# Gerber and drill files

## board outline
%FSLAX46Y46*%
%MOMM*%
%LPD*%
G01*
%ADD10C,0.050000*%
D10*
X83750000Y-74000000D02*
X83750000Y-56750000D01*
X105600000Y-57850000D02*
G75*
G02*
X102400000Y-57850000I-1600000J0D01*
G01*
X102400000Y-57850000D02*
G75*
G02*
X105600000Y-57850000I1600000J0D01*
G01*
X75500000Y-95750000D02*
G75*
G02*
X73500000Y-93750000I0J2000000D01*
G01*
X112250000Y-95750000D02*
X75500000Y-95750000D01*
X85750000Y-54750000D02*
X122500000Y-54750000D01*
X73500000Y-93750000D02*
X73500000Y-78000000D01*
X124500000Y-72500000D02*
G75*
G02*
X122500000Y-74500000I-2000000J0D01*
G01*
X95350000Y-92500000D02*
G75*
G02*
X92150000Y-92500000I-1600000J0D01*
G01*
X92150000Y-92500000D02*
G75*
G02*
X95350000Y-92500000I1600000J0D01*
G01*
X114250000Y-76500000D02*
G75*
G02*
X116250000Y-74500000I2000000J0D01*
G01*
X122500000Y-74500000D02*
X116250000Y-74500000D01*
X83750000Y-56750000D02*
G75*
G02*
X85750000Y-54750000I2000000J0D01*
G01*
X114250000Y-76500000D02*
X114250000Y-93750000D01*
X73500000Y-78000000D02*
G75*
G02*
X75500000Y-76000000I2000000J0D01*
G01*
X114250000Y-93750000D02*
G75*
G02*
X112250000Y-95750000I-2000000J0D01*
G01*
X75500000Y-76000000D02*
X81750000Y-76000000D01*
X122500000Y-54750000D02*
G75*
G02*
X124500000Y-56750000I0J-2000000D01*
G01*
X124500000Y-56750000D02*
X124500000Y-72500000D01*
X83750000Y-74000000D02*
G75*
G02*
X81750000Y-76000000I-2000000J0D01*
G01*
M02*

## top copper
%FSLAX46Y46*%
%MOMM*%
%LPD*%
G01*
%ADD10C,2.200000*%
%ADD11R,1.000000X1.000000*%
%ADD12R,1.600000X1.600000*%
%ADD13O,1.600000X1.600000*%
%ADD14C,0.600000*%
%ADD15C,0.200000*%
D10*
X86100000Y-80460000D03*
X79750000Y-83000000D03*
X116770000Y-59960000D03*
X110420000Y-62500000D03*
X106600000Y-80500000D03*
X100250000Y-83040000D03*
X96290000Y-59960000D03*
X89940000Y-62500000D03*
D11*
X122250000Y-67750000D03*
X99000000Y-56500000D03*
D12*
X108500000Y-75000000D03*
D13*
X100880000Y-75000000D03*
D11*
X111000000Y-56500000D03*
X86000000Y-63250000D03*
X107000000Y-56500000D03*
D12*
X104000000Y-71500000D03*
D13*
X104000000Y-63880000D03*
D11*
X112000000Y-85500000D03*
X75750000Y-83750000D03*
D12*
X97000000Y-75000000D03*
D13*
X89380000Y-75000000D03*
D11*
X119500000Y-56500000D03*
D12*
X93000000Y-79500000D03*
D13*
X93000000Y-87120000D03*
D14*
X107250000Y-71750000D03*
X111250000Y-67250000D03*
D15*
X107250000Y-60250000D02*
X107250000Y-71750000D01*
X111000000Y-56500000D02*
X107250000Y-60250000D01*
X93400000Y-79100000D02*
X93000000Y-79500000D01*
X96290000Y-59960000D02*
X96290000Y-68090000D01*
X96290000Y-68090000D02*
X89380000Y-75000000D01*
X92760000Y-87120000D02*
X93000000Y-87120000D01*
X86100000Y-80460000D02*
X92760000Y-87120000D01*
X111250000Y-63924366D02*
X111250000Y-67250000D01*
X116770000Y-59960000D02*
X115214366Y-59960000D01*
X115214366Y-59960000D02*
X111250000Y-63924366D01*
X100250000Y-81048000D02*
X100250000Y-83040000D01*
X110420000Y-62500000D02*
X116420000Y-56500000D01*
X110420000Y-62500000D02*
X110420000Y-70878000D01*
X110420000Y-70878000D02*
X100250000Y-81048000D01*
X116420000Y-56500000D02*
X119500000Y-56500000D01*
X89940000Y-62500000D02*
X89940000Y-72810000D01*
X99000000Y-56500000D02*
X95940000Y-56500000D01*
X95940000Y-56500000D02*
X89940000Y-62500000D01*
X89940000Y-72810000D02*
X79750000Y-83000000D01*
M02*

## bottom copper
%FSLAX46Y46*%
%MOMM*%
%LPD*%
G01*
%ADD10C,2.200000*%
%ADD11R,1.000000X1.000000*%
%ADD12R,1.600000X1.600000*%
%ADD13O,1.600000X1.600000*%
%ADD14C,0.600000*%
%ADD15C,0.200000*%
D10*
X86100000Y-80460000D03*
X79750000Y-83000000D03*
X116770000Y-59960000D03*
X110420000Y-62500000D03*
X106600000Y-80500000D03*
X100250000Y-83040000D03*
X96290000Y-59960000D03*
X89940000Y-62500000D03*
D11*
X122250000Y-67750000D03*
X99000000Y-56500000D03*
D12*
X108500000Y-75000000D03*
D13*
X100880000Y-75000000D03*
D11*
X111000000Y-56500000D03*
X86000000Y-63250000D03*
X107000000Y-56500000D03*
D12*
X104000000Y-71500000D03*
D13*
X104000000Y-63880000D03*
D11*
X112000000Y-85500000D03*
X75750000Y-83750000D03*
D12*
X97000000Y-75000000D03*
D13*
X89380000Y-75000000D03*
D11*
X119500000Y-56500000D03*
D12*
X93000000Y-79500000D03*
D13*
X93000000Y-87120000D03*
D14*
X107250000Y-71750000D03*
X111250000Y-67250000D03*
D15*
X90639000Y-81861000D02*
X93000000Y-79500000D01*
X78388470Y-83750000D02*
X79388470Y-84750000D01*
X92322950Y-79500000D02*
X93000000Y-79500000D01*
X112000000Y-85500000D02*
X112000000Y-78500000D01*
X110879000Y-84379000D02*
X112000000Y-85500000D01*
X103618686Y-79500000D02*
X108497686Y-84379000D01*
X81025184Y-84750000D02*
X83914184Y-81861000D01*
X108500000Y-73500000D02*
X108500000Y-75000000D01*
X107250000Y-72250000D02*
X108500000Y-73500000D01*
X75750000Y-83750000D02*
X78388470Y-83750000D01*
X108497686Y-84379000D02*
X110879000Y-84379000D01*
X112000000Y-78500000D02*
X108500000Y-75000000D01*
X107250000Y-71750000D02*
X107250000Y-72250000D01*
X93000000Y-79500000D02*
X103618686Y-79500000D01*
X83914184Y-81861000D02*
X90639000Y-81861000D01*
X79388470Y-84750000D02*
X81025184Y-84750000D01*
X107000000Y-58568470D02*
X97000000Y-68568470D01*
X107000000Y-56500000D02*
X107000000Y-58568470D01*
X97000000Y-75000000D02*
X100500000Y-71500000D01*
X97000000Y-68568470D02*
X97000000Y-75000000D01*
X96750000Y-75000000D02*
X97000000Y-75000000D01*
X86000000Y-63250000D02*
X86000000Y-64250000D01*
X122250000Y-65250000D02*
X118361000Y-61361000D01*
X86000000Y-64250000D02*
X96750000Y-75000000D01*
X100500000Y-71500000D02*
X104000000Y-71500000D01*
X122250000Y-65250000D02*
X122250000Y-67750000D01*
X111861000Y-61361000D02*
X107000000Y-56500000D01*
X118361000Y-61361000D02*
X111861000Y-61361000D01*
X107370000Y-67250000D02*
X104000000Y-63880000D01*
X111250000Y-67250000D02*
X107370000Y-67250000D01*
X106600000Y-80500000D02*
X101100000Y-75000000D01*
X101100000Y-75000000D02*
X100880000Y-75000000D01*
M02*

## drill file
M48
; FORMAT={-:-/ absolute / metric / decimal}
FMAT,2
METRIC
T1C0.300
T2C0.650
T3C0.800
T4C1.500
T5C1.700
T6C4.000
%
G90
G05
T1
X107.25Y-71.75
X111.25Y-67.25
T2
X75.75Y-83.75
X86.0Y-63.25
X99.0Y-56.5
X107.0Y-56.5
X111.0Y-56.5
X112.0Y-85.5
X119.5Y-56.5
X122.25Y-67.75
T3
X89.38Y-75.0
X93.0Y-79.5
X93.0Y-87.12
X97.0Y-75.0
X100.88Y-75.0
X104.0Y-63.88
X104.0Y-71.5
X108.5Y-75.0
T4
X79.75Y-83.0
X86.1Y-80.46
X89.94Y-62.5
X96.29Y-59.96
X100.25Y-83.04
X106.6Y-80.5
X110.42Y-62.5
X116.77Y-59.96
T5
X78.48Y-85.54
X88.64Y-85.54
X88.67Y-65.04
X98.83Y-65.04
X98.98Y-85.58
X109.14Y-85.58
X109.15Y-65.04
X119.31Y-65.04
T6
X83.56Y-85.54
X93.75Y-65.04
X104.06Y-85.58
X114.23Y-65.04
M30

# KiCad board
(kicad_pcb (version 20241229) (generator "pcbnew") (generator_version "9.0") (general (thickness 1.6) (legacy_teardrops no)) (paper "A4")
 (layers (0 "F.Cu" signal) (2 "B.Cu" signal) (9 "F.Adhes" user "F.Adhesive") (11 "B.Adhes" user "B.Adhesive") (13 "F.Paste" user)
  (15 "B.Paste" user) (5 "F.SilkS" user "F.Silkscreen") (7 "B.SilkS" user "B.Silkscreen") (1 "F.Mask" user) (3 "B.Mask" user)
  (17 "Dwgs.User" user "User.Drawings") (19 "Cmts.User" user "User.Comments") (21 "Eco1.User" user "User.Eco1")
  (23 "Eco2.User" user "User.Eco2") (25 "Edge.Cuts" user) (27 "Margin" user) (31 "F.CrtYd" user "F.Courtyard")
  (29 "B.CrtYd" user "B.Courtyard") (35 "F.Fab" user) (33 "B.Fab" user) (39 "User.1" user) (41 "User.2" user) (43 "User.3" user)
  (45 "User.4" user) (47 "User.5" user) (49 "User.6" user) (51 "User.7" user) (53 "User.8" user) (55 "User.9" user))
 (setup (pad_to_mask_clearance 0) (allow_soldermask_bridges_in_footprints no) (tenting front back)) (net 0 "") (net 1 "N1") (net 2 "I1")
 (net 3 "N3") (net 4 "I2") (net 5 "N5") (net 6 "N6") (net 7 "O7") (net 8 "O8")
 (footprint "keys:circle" (layer "F.Cu") (at 94 65)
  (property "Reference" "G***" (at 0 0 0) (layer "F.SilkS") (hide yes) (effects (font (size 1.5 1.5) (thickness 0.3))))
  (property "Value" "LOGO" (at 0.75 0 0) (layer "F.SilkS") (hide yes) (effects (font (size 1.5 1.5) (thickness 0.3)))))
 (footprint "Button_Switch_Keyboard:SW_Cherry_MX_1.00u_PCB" (layer "F.Cu") (at 86.1 80.46)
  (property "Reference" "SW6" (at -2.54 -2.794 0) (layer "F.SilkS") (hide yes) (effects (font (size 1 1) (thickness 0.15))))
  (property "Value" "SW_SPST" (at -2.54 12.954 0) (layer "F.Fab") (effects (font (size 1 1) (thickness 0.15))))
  (pad "" np_thru_hole circle (at -7.62 5.08) (size 1.7 1.7) (drill 1.7) (layers "*.Cu" "*.Mask"))
  (pad "" np_thru_hole circle (at -2.54 5.08) (size 4 4) (drill 4) (layers "*.Cu" "*.Mask"))
  (pad "" np_thru_hole circle (at 2.54 5.08) (size 1.7 1.7) (drill 1.7) (layers "*.Cu" "*.Mask"))
  (pad "1" thru_hole circle (at 0 0) (size 2.2 2.2) (drill 1.5) (layers "*.Cu" "*.Mask") (remove_unused_layers no) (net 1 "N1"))
  (pad "2" thru_hole circle (at -6.35 2.54) (size 2.2 2.2) (drill 1.5) (layers "*.Cu" "*.Mask") (remove_unused_layers no) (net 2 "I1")))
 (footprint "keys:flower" (layer "F.Cu") (at 114.2 65)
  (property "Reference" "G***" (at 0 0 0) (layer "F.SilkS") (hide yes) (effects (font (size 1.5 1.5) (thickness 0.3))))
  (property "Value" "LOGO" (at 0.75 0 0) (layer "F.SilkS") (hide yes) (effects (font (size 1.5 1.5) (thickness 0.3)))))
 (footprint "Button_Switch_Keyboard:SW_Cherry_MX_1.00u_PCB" (layer "F.Cu") (at 116.77 59.96)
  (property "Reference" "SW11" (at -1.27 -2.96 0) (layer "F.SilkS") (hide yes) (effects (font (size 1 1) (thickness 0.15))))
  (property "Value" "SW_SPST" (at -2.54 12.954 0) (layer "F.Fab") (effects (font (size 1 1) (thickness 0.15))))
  (pad "" np_thru_hole circle (at -7.62 5.08) (size 1.7 1.7) (drill 1.7) (layers "*.Cu" "*.Mask"))
  (pad "" np_thru_hole circle (at -2.54 5.08) (size 4 4) (drill 4) (layers "*.Cu" "*.Mask"))
  (pad "" np_thru_hole circle (at 2.54 5.08) (size 1.7 1.7) (drill 1.7) (layers "*.Cu" "*.Mask"))
  (pad "1" thru_hole circle (at 0 0) (size 2.2 2.2) (drill 1.5) (layers "*.Cu" "*.Mask") (remove_unused_layers no) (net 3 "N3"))
  (pad "2" thru_hole circle (at -6.35 2.54) (size 2.2 2.2) (drill 1.5) (layers "*.Cu" "*.Mask") (remove_unused_layers no) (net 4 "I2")))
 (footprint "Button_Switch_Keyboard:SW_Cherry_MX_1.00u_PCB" (layer "F.Cu") (at 106.6 80.5)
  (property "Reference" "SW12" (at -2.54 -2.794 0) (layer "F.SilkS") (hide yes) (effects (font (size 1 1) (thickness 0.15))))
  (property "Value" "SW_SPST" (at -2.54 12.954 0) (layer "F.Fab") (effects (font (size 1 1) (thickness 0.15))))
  (pad "" np_thru_hole circle (at -7.62 5.08) (size 1.7 1.7) (drill 1.7) (layers "*.Cu" "*.Mask"))
  (pad "" np_thru_hole circle (at -2.54 5.08) (size 4 4) (drill 4) (layers "*.Cu" "*.Mask"))
  (pad "" np_thru_hole circle (at 2.54 5.08) (size 1.7 1.7) (drill 1.7) (layers "*.Cu" "*.Mask"))
  (pad "1" thru_hole circle (at 0 0) (size 2.2 2.2) (drill 1.5) (layers "*.Cu" "*.Mask") (remove_unused_layers no) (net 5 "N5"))
  (pad "2" thru_hole circle (at -6.35 2.54) (size 2.2 2.2) (drill 1.5) (layers "*.Cu" "*.Mask") (remove_unused_layers no) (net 4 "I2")))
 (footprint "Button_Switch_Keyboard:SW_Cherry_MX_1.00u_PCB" (layer "F.Cu") (at 96.29 59.96)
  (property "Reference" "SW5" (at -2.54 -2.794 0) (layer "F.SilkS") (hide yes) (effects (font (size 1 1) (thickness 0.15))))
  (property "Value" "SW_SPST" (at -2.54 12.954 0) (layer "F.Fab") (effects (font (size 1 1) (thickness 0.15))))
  (pad "" np_thru_hole circle (at -7.62 5.08) (size 1.7 1.7) (drill 1.7) (layers "*.Cu" "*.Mask"))
  (pad "" np_thru_hole circle (at -2.54 5.08) (size 4 4) (drill 4) (layers "*.Cu" "*.Mask"))
  (pad "" np_thru_hole circle (at 2.54 5.08) (size 1.7 1.7) (drill 1.7) (layers "*.Cu" "*.Mask"))
  (pad "1" thru_hole circle (at 0 0) (size 2.2 2.2) (drill 1.5) (layers "*.Cu" "*.Mask") (remove_unused_layers no) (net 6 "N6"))
  (pad "2" thru_hole circle (at -6.35 2.54) (size 2.2 2.2) (drill 1.5) (layers "*.Cu" "*.Mask") (remove_unused_layers no) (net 2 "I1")))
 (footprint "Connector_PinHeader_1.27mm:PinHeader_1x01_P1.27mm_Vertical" (layer "B.Cu") (at 122.25 67.75)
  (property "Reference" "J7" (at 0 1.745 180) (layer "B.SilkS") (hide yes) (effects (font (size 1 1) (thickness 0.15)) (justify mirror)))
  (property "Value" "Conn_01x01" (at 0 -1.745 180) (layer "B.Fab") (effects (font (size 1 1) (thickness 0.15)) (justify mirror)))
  (pad "1" thru_hole rect (at 0 0) (size 1 1) (drill 0.65) (layers "*.Cu" "*.Mask") (remove_unused_layers no) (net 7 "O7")))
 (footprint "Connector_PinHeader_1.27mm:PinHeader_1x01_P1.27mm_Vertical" (layer "B.Cu") (at 99 56.5)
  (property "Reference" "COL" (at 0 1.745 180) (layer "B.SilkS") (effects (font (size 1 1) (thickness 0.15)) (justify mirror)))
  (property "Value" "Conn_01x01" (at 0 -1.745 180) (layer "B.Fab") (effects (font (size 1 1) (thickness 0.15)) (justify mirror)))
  (pad "1" thru_hole rect (at 0 0) (size 1 1) (drill 0.65) (layers "*.Cu" "*.Mask") (remove_unused_layers no) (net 2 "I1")))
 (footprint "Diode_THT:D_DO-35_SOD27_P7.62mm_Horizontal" (layer "B.Cu") (at 108.5 75 180)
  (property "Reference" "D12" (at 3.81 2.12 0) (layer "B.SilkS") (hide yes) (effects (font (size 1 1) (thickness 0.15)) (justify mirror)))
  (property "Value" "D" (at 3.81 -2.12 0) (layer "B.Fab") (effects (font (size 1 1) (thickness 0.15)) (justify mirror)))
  (pad "1" thru_hole rect (at 0 0 180) (size 1.6 1.6) (drill 0.8) (layers "*.Cu" "*.Mask") (remove_unused_layers no) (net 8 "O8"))
  (pad "2" thru_hole oval (at 7.62 0 180) (size 1.6 1.6) (drill 0.8) (layers "*.Cu" "*.Mask") (remove_unused_layers no) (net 5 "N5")))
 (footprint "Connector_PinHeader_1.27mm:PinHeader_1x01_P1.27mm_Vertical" (layer "B.Cu") (at 111 56.5)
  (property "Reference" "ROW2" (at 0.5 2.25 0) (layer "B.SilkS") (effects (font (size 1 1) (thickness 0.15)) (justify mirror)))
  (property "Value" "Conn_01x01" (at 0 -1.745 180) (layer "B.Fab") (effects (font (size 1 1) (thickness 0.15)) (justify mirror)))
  (pad "1" thru_hole rect (at 0 0) (size 1 1) (drill 0.65) (layers "*.Cu" "*.Mask") (remove_unused_layers no) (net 8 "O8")))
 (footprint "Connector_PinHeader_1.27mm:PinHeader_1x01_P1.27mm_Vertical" (layer "B.Cu") (at 86 63.25)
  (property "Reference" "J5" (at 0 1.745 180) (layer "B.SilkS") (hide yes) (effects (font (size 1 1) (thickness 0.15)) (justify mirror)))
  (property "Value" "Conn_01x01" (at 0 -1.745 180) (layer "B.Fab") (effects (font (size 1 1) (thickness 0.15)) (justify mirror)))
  (pad "1" thru_hole rect (at 0 0) (size 1 1) (drill 0.65) (layers "*.Cu" "*.Mask") (remove_unused_layers no) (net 7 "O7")))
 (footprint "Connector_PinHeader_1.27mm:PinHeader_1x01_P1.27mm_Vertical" (layer "B.Cu") (at 107 56.5)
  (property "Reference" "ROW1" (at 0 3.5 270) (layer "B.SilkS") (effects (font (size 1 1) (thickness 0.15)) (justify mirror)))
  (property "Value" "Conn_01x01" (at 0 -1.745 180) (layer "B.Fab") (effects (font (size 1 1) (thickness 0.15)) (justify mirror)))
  (pad "1" thru_hole rect (at 0 0) (size 1 1) (drill 0.65) (layers "*.Cu" "*.Mask") (remove_unused_layers no) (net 7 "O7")))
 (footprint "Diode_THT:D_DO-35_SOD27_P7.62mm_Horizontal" (layer "B.Cu") (at 104 71.5 90)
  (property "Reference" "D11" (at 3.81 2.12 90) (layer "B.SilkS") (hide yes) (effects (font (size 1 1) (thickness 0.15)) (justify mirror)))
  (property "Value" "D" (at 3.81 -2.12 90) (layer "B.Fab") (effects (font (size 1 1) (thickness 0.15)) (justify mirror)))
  (pad "1" thru_hole rect (at 0 0 90) (size 1.6 1.6) (drill 0.8) (layers "*.Cu" "*.Mask") (remove_unused_layers no) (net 7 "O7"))
  (pad "2" thru_hole oval (at 7.62 0 90) (size 1.6 1.6) (drill 0.8) (layers "*.Cu" "*.Mask") (remove_unused_layers no) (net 3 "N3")))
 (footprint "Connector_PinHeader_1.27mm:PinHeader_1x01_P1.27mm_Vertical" (layer "B.Cu") (at 112 85.5)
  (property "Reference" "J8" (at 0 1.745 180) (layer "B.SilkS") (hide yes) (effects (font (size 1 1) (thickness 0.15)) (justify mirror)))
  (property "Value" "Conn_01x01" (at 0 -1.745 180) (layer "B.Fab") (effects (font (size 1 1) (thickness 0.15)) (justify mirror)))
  (pad "1" thru_hole rect (at 0 0) (size 1 1) (drill 0.65) (layers "*.Cu" "*.Mask") (remove_unused_layers no) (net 8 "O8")))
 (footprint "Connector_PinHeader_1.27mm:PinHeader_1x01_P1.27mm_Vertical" (layer "B.Cu") (at 75.75 83.75)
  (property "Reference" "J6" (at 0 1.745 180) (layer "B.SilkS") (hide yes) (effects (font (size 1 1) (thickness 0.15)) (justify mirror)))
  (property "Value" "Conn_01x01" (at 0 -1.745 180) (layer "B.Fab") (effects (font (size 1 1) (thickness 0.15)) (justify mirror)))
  (pad "1" thru_hole rect (at 0 0) (size 1 1) (drill 0.65) (layers "*.Cu" "*.Mask") (remove_unused_layers no) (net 8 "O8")))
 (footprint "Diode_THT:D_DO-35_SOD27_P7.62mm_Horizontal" (layer "B.Cu") (at 97 75 180)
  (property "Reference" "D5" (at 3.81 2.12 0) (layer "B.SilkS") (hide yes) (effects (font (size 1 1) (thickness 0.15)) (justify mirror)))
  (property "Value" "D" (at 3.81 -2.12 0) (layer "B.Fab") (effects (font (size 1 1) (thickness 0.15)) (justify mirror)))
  (pad "1" thru_hole rect (at 0 0 180) (size 1.6 1.6) (drill 0.8) (layers "*.Cu" "*.Mask") (remove_unused_layers no) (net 7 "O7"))
  (pad "2" thru_hole oval (at 7.62 0 180) (size 1.6 1.6) (drill 0.8) (layers "*.Cu" "*.Mask") (remove_unused_layers no) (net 6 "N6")))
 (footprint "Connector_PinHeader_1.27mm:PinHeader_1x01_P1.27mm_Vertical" (layer "B.Cu") (at 119.5 56.5)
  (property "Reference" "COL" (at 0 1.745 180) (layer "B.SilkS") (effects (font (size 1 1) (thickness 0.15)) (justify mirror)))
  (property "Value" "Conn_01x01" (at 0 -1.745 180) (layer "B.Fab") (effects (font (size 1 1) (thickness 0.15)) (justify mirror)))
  (pad "1" thru_hole rect (at 0 0) (size 1 1) (drill 0.65) (layers "*.Cu" "*.Mask") (remove_unused_layers no) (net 4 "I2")))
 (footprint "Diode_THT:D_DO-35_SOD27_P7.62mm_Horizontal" (layer "B.Cu") (at 93 79.5 -90)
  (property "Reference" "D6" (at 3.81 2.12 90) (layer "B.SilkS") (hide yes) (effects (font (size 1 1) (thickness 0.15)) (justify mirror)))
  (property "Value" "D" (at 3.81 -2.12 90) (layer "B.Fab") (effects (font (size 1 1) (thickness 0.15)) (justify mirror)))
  (pad "1" thru_hole rect (at 0 0 270) (size 1.6 1.6) (drill 0.8) (layers "*.Cu" "*.Mask") (remove_unused_layers no) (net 8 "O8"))
  (pad "2" thru_hole oval (at 7.62 0 270) (size 1.6 1.6) (drill 0.8) (layers "*.Cu" "*.Mask") (remove_unused_layers no) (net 1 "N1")))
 (gr_line (start 83.75 74) (end 83.75 56.75) (stroke (width 0.05) (type default)) (layer "Edge.Cuts"))
 (gr_circle (center 104 57.85) (end 105.6 57.85) (stroke (width 0.05) (type solid)) (fill no) (layer "Edge.Cuts"))
 (gr_arc (start 75.5 95.75) (mid 74.085786 95.164214) (end 73.5 93.75) (stroke (width 0.05) (type default)) (layer "Edge.Cuts"))
 (gr_line (start 112.25 95.75) (end 75.5 95.75) (stroke (width 0.05) (type default)) (layer "Edge.Cuts"))
 (gr_line (start 85.75 54.75) (end 122.5 54.75) (stroke (width 0.05) (type default)) (layer "Edge.Cuts"))
 (gr_line (start 73.5 93.75) (end 73.5 78) (stroke (width 0.05) (type default)) (layer "Edge.Cuts"))
 (gr_arc (start 124.5 72.5) (mid 123.914214 73.914214) (end 122.5 74.5) (stroke (width 0.05) (type default)) (layer "Edge.Cuts"))
 (gr_circle (center 93.75 92.5) (end 95.35 92.5) (stroke (width 0.05) (type solid)) (fill no) (layer "Edge.Cuts"))
 (gr_arc (start 114.25 76.5) (mid 114.835786 75.085786) (end 116.25 74.5) (stroke (width 0.05) (type default)) (layer "Edge.Cuts"))
 (gr_line (start 122.5 74.5) (end 116.25 74.5) (stroke (width 0.05) (type default)) (layer "Edge.Cuts"))
 (gr_arc (start 83.75 56.75) (mid 84.335786 55.335786) (end 85.75 54.75) (stroke (width 0.05) (type default)) (layer "Edge.Cuts"))
 (gr_line (start 114.25 76.5) (end 114.25 93.75) (stroke (width 0.05) (type default)) (layer "Edge.Cuts"))
 (gr_arc (start 73.5 78) (mid 74.085786 76.585786) (end 75.5 76) (stroke (width 0.05) (type default)) (layer "Edge.Cuts"))
 (gr_arc (start 114.25 93.75) (mid 113.664214 95.164214) (end 112.25 95.75) (stroke (width 0.05) (type default)) (layer "Edge.Cuts"))
 (gr_line (start 75.5 76) (end 81.75 76) (stroke (width 0.05) (type default)) (layer "Edge.Cuts"))
 (gr_arc (start 122.5 54.75) (mid 123.914214 55.335786) (end 124.5 56.75) (stroke (width 0.05) (type default)) (layer "Edge.Cuts"))
 (gr_line (start 124.5 56.75) (end 124.5 72.5) (stroke (width 0.05) (type default)) (layer "Edge.Cuts"))
 (gr_arc (start 83.75 74) (mid 83.164214 75.414214) (end 81.75 76) (stroke (width 0.05) (type default)) (layer "Edge.Cuts"))
 (segment (start 107.25 60.25) (end 107.25 71.75) (width 0.2) (layer "F.Cu") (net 8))
 (segment (start 111 56.5) (end 107.25 60.25) (width 0.2) (layer "F.Cu") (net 8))
 (segment (start 93.4 79.1) (end 93 79.5) (width 0.2) (layer "F.Cu") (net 8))
 (via (at 107.25 71.75) (size 0.6) (drill 0.3) (layers "F.Cu" "B.Cu") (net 8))
 (segment (start 90.639 81.861) (end 93 79.5) (width 0.2) (layer "B.Cu") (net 8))
 (segment (start 78.38847 83.75) (end 79.38847 84.75) (width 0.2) (layer "B.Cu") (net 8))
 (segment (start 92.32295 79.5) (end 93 79.5) (width 0.2) (layer "B.Cu") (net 8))
 (segment (start 112 85.5) (end 112 78.5) (width 0.2) (layer "B.Cu") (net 8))
 (segment (start 110.879 84.379) (end 112 85.5) (width 0.2) (layer "B.Cu") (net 8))
 (segment (start 103.618686 79.5) (end 108.497686 84.379) (width 0.2) (layer "B.Cu") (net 8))
 (segment (start 81.025184 84.75) (end 83.914184 81.861) (width 0.2) (layer "B.Cu") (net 8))
 (segment (start 108.5 73.5) (end 108.5 75) (width 0.2) (layer "B.Cu") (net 8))
 (segment (start 107.25 72.25) (end 108.5 73.5) (width 0.2) (layer "B.Cu") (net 8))
 (segment (start 75.75 83.75) (end 78.38847 83.75) (width 0.2) (layer "B.Cu") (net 8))
 (segment (start 108.497686 84.379) (end 110.879 84.379) (width 0.2) (layer "B.Cu") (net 8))
 (segment (start 112 78.5) (end 108.5 75) (width 0.2) (layer "B.Cu") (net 8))
 (segment (start 107.25 71.75) (end 107.25 72.25) (width 0.2) (layer "B.Cu") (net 8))
 (segment (start 93 79.5) (end 103.618686 79.5) (width 0.2) (layer "B.Cu") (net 8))
 (segment (start 83.914184 81.861) (end 90.639 81.861) (width 0.2) (layer "B.Cu") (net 8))
 (segment (start 79.38847 84.75) (end 81.025184 84.75) (width 0.2) (layer "B.Cu") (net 8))
 (segment (start 96.29 59.96) (end 96.29 68.09) (width 0.2) (layer "F.Cu") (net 6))
 (segment (start 96.29 68.09) (end 89.38 75) (width 0.2) (layer "F.Cu") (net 6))
 (segment (start 107 58.56847) (end 97 68.56847) (width 0.2) (layer "B.Cu") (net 7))
 (segment (start 107 56.5) (end 107 58.56847) (width 0.2) (layer "B.Cu") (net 7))
 (segment (start 97 75) (end 100.5 71.5) (width 0.2) (layer "B.Cu") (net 7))
 (segment (start 97 68.56847) (end 97 75) (width 0.2) (layer "B.Cu") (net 7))
 (segment (start 96.75 75) (end 97 75) (width 0.2) (layer "B.Cu") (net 7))
 (segment (start 86 63.25) (end 86 64.25) (width 0.2) (layer "B.Cu") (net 7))
 (segment (start 122.25 65.25) (end 118.361 61.361) (width 0.2) (layer "B.Cu") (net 7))
 (segment (start 86 64.25) (end 96.75 75) (width 0.2) (layer "B.Cu") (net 7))
 (segment (start 100.5 71.5) (end 104 71.5) (width 0.2) (layer "B.Cu") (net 7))
 (segment (start 122.25 65.25) (end 122.25 67.75) (width 0.2) (layer "B.Cu") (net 7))
 (segment (start 111.861 61.361) (end 107 56.5) (width 0.2) (layer "B.Cu") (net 7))
 (segment (start 118.361 61.361) (end 111.861 61.361) (width 0.2) (layer "B.Cu") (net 7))
 (segment (start 92.76 87.12) (end 93 87.12) (width 0.2) (layer "F.Cu") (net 1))
 (segment (start 86.1 80.46) (end 92.76 87.12) (width 0.2) (layer "F.Cu") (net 1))
 (segment (start 111.25 63.924366) (end 111.25 67.25) (width 0.2) (layer "F.Cu") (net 3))
 (segment (start 116.77 59.96) (end 115.214366 59.96) (width 0.2) (layer "F.Cu") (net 3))
 (segment (start 115.214366 59.96) (end 111.25 63.924366) (width 0.2) (layer "F.Cu") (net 3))
 (via (at 111.25 67.25) (size 0.6) (drill 0.3) (layers "F.Cu" "B.Cu") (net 3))
 (segment (start 107.37 67.25) (end 104 63.88) (width 0.2) (layer "B.Cu") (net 3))
 (segment (start 111.25 67.25) (end 107.37 67.25) (width 0.2) (layer "B.Cu") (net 3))
 (segment (start 106.6 80.5) (end 101.1 75) (width 0.2) (layer "B.Cu") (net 5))
 (segment (start 101.1 75) (end 100.88 75) (width 0.2) (layer "B.Cu") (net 5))
 (segment (start 100.25 81.048) (end 100.25 83.04) (width 0.2) (layer "F.Cu") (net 4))
 (segment (start 110.42 62.5) (end 116.42 56.5) (width 0.2) (layer "F.Cu") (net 4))
 (segment (start 110.42 62.5) (end 110.42 70.878) (width 0.2) (layer "F.Cu") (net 4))
 (segment (start 110.42 70.878) (end 100.25 81.048) (width 0.2) (layer "F.Cu") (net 4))
 (segment (start 116.42 56.5) (end 119.5 56.5) (width 0.2) (layer "F.Cu") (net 4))
 (segment (start 89.94 62.5) (end 89.94 72.81) (width 0.2) (layer "F.Cu") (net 2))
 (segment (start 99 56.5) (end 95.94 56.5) (width 0.2) (layer "F.Cu") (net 2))
 (segment (start 95.94 56.5) (end 89.94 62.5) (width 0.2) (layer "F.Cu") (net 2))
 (segment (start 89.94 72.81) (end 79.75 83) (width 0.2) (layer "F.Cu") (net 2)))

